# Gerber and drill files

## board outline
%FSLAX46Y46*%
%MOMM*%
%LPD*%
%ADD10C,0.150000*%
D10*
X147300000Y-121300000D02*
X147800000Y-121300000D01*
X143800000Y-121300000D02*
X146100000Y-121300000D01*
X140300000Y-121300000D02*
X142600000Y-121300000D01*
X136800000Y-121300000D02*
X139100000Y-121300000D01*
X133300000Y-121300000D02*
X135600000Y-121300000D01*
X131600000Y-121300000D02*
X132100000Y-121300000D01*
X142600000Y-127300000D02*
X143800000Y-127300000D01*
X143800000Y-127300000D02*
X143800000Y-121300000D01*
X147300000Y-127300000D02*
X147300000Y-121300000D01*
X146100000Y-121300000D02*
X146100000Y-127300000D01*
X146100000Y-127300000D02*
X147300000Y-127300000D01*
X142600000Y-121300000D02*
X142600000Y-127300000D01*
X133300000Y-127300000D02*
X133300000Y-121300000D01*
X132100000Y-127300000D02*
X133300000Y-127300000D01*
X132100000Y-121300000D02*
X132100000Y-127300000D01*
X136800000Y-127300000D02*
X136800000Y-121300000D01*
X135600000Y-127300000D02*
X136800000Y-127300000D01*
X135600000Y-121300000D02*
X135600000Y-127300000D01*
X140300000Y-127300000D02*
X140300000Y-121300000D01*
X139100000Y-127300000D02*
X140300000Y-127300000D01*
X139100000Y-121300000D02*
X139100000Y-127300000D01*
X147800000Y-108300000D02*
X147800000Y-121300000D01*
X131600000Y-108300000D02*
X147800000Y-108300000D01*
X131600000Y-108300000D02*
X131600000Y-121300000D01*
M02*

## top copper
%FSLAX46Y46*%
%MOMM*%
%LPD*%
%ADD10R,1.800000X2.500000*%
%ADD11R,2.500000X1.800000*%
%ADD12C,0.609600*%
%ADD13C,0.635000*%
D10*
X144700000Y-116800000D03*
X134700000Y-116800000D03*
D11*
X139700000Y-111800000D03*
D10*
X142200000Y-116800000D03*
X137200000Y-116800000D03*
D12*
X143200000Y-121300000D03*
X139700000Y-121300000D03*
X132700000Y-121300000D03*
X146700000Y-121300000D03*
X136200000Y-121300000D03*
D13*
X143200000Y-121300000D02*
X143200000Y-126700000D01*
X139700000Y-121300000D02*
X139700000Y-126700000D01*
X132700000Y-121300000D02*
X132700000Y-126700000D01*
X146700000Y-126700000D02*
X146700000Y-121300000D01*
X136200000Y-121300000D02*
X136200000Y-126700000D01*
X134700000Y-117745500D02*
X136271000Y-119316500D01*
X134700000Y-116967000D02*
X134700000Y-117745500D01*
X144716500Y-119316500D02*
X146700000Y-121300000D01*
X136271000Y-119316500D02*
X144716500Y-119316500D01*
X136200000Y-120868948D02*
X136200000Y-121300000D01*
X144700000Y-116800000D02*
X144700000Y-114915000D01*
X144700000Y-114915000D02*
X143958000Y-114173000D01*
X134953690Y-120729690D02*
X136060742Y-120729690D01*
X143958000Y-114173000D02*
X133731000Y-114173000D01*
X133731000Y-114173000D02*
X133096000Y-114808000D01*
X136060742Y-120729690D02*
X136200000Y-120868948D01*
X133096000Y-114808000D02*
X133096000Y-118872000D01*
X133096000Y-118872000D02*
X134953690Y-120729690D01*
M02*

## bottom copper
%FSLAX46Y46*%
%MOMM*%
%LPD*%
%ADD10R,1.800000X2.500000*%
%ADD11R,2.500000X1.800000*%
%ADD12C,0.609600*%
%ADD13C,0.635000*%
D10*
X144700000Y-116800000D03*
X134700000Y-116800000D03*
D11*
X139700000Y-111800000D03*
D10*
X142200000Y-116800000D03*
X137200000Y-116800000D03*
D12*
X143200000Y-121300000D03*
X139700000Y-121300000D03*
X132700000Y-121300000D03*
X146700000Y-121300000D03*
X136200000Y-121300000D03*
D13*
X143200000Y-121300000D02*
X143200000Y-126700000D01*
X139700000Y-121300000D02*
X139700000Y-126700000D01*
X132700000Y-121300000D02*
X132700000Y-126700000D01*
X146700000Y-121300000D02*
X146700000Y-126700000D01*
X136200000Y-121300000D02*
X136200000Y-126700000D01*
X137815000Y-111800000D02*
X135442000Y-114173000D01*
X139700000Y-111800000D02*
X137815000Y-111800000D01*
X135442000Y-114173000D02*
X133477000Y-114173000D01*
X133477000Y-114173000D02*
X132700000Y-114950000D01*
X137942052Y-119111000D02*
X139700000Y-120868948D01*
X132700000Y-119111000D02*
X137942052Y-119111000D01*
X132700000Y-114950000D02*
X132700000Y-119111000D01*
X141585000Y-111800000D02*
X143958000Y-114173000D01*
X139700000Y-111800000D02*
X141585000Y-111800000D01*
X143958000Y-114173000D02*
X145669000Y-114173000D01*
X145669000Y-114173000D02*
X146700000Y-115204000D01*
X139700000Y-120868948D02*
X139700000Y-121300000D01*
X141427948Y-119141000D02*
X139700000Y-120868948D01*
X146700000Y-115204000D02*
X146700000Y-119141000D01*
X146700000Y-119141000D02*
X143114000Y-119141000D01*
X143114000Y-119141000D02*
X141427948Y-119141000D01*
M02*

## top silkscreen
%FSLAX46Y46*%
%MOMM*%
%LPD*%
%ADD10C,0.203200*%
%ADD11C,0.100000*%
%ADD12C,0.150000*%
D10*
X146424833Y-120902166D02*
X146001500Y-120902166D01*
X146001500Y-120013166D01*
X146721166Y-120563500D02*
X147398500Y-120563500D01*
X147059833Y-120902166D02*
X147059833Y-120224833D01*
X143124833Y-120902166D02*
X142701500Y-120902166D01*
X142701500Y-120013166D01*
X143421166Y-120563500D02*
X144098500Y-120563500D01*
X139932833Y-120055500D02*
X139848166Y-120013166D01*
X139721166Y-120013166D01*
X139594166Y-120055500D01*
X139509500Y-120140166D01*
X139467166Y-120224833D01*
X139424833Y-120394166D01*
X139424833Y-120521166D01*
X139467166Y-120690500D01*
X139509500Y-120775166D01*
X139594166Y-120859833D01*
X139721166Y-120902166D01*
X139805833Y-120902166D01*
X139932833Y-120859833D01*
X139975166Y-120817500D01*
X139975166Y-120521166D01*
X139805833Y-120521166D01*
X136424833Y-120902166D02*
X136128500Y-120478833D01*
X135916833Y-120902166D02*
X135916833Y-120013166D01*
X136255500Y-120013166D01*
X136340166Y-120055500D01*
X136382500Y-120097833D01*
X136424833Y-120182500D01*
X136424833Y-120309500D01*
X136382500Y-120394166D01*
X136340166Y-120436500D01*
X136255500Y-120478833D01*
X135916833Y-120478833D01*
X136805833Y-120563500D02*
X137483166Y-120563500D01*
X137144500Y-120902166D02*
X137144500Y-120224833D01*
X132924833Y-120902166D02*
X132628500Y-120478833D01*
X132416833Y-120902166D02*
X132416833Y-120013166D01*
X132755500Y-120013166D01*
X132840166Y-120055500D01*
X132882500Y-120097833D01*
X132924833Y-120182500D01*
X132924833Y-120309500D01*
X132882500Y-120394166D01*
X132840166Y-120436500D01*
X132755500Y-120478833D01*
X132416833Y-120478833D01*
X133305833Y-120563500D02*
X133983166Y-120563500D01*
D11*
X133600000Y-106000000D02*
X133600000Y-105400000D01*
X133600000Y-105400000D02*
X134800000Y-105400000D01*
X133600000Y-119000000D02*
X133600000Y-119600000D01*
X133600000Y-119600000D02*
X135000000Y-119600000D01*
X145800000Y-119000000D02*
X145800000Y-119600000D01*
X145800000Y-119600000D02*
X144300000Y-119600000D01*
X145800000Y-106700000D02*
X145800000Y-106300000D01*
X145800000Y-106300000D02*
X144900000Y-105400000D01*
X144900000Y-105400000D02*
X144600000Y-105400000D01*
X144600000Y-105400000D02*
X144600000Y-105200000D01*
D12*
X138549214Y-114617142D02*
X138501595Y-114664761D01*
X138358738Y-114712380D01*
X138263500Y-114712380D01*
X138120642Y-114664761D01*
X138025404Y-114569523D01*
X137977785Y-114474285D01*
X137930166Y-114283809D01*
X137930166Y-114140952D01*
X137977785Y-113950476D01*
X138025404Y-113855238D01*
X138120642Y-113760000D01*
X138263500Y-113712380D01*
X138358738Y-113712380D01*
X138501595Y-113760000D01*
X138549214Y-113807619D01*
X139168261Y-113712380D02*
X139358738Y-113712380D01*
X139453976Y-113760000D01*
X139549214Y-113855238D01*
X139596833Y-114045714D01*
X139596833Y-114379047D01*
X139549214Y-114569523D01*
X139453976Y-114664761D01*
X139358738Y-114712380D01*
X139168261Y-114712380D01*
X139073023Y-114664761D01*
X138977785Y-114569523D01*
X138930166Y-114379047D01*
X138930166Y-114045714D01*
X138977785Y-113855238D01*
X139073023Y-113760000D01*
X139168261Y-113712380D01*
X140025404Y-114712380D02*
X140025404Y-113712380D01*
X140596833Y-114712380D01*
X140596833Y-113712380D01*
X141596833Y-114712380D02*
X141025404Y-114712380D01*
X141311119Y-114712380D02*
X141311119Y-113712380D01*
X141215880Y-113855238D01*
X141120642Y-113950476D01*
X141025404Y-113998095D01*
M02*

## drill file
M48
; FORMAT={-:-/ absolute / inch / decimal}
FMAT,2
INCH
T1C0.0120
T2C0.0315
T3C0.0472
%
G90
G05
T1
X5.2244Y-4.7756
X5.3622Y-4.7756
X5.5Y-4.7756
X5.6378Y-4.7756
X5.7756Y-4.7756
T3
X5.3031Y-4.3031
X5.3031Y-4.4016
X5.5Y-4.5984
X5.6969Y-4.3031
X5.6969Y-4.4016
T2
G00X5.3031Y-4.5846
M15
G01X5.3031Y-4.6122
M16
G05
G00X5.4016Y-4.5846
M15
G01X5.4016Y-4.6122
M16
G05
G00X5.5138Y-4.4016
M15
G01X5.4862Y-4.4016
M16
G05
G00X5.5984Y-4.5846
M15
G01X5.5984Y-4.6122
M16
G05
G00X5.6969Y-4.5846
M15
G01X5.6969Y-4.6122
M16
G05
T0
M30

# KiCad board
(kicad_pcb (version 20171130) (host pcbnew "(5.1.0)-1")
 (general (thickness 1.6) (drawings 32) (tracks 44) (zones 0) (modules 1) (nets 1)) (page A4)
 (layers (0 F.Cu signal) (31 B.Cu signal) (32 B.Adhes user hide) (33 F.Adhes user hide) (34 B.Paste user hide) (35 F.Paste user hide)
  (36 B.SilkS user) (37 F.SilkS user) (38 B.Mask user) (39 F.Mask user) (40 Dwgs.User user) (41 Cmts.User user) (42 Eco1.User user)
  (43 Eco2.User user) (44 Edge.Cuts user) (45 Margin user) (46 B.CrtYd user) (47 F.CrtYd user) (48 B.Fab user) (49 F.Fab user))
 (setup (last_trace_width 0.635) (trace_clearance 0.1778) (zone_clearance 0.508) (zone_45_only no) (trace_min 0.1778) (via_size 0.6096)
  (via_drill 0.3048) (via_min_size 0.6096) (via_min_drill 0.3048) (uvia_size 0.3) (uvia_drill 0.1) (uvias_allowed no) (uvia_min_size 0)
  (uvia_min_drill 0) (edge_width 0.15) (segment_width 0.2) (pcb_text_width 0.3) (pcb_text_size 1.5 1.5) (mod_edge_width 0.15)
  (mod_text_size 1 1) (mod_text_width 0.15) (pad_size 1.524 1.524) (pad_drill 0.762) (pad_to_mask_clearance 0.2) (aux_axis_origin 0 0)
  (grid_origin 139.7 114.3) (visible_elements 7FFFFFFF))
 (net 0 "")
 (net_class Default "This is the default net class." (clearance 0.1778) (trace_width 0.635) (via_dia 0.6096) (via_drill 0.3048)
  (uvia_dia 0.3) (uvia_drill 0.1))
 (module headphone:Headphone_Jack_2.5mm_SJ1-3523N (layer F.Cu) (at 139.7 116.8 270)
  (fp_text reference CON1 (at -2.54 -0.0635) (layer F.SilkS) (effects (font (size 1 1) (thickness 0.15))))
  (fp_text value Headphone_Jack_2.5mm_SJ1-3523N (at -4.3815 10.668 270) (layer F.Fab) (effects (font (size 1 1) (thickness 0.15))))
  (fp_line (start -10.8 6.1) (end -11.4 6.1) (layer F.SilkS) (width 0.1))
  (fp_line (start -11.4 6.1) (end -11.4 4.9) (layer F.SilkS) (width 0.1))
  (fp_line (start 2.2 6.1) (end 2.8 6.1) (layer F.SilkS) (width 0.1))
  (fp_line (start 2.8 6.1) (end 2.8 4.7) (layer F.SilkS) (width 0.1))
  (fp_line (start 2.2 -6.1) (end 2.8 -6.1) (layer F.SilkS) (width 0.1))
  (fp_line (start 2.8 -6.1) (end 2.8 -4.6) (layer F.SilkS) (width 0.1))
  (fp_line (start -10.1 -6.1) (end -10.5 -6.1) (layer F.SilkS) (width 0.1))
  (fp_line (start -10.5 -6.1) (end -11.4 -5.2) (layer F.SilkS) (width 0.1))
  (fp_line (start -11.4 -5.2) (end -11.4 -4.9) (layer F.SilkS) (width 0.1))
  (fp_line (start -11.4 -4.9) (end -11.6 -4.9) (layer F.SilkS) (width 0.1))
  (pad 3 thru_hole rect (at 0 -5 270) (size 2.5 1.8) (drill oval 1.5 0.8) (layers *.Cu *.Mask))
  (pad 2 thru_hole rect (at 0 5 270) (size 2.5 1.8) (drill oval 1.5 0.8) (layers *.Cu *.Mask))
  (pad 1 thru_hole rect (at -5 0 270) (size 1.8 2.5) (drill oval 0.8 1.5) (layers *.Cu *.Mask))
  (pad "" np_thru_hole circle (at 0 0 270) (size 1.2 1.2) (drill 1.2) (layers *.Cu *.Mask))
  (pad "" np_thru_hole circle (at -5 -5 270) (size 1.2 1.2) (drill 1.2) (layers *.Cu *.Mask))
  (pad "" np_thru_hole circle (at -7.5 -5 270) (size 1.2 1.2) (drill 1.2) (layers *.Cu *.Mask))
  (pad "" np_thru_hole circle (at -5 5 270) (size 1.2 1.2) (drill 1.2) (layers *.Cu *.Mask))
  (pad "" np_thru_hole circle (at -7.5 5 270) (size 1.2 1.2) (drill 1.2) (layers *.Cu *.Mask))
  (pad 11 thru_hole rect (at 0 -2.5 270) (size 2.5 1.8) (drill oval 1.5 0.8) (layers *.Cu *.Mask))
  (pad 10 thru_hole rect (at 0 2.5 270) (size 2.5 1.8) (drill oval 1.5 0.8) (layers *.Cu *.Mask)))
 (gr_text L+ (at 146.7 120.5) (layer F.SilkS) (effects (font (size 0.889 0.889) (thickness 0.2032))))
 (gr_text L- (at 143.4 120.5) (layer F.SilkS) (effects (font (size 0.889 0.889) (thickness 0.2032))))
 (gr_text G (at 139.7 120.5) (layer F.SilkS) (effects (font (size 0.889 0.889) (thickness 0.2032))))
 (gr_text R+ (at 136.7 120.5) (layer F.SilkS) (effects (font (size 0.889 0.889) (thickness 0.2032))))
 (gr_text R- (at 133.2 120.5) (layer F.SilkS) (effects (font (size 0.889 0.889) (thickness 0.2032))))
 (gr_line (start 147.3 121.3) (end 147.8 121.3) (layer Edge.Cuts) (width 0.15))
 (gr_line (start 143.8 121.3) (end 146.1 121.3) (layer Edge.Cuts) (width 0.15))
 (gr_line (start 140.3 121.3) (end 142.6 121.3) (layer Edge.Cuts) (width 0.15))
 (gr_line (start 136.8 121.3) (end 139.1 121.3) (layer Edge.Cuts) (width 0.15))
 (gr_line (start 133.3 121.3) (end 135.6 121.3) (layer Edge.Cuts) (width 0.15))
 (gr_line (start 131.6 121.3) (end 132.1 121.3) (layer Edge.Cuts) (width 0.15))
 (gr_line (start 142.6 127.3) (end 143.8 127.3) (layer Edge.Cuts) (width 0.15))
 (gr_line (start 143.8 127.3) (end 143.8 121.3) (layer Edge.Cuts) (width 0.15))
 (gr_line (start 147.3 127.3) (end 147.3 121.3) (layer Edge.Cuts) (width 0.15))
 (gr_line (start 146.1 121.3) (end 146.1 127.3) (layer Edge.Cuts) (width 0.15))
 (gr_line (start 146.1 127.3) (end 147.3 127.3) (layer Edge.Cuts) (width 0.15))
 (gr_line (start 142.6 121.3) (end 142.6 127.3) (layer Edge.Cuts) (width 0.15))
 (gr_line (start 133.3 127.3) (end 133.3 121.3) (layer Edge.Cuts) (width 0.15))
 (gr_line (start 132.1 127.3) (end 133.3 127.3) (layer Edge.Cuts) (width 0.15))
 (gr_line (start 132.1 121.3) (end 132.1 127.3) (layer Edge.Cuts) (width 0.15))
 (gr_line (start 136.8 127.3) (end 136.8 121.3) (layer Edge.Cuts) (width 0.15))
 (gr_line (start 135.6 127.3) (end 136.8 127.3) (layer Edge.Cuts) (width 0.15))
 (gr_line (start 135.6 121.3) (end 135.6 127.3) (layer Edge.Cuts) (width 0.15))
 (gr_line (start 140.3 127.3) (end 140.3 121.3) (layer Edge.Cuts) (width 0.15))
 (gr_line (start 139.1 127.3) (end 140.3 127.3) (layer Edge.Cuts) (width 0.15))
 (gr_line (start 139.1 121.3) (end 139.1 127.3) (layer Edge.Cuts) (width 0.15))
 (gr_line (start 147.8 108.3) (end 147.8 121.3) (layer Edge.Cuts) (width 0.15))
 (gr_line (start 131.6 108.3) (end 147.8 108.3) (layer Edge.Cuts) (width 0.15))
 (gr_line (start 131.6 108.3) (end 131.6 121.3) (layer Edge.Cuts) (width 0.15))
 (segment (start 143.2 121.3) (end 143.2 126.7) (width 0.635) (layer F.Cu) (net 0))
 (via (at 143.2 121.3) (size 0.6096) (drill 0.3048) (layers F.Cu B.Cu) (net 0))
 (segment (start 143.2 121.3) (end 143.2 126.7) (width 0.635) (layer B.Cu) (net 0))
 (segment (start 139.7 121.3) (end 139.7 126.7) (width 0.635) (layer F.Cu) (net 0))
 (segment (start 139.7 121.3) (end 139.7 126.7) (width 0.635) (layer B.Cu) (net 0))
 (via (at 139.7 121.3) (size 0.6096) (drill 0.3048) (layers F.Cu B.Cu) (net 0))
 (segment (start 132.7 121.3) (end 132.7 126.7) (width 0.635) (layer F.Cu) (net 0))
 (segment (start 132.7 121.3) (end 132.7 126.7) (width 0.635) (layer B.Cu) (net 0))
 (via (at 132.7 121.3) (size 0.6096) (drill 0.3048) (layers F.Cu B.Cu) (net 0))
 (segment (start 146.7 121.3) (end 146.7 126.7) (width 0.635) (layer B.Cu) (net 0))
 (segment (start 146.7 126.7) (end 146.7 121.3) (width 0.635) (layer F.Cu) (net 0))
 (via (at 146.7 121.3) (size 0.6096) (drill 0.3048) (layers F.Cu B.Cu) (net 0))
 (segment (start 136.2 121.3) (end 136.2 126.7) (width 0.635) (layer B.Cu) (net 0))
 (segment (start 136.2 121.3) (end 136.2 126.7) (width 0.635) (layer F.Cu) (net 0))
 (via (at 136.2 121.3) (size 0.6096) (drill 0.3048) (layers F.Cu B.Cu) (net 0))
 (segment (start 134.7 117.7455) (end 136.271 119.3165) (width 0.635) (layer F.Cu) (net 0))
 (segment (start 134.7 116.967) (end 134.7 117.7455) (width 0.635) (layer F.Cu) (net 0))
 (segment (start 144.7165 119.3165) (end 146.7 121.3) (width 0.635) (layer F.Cu) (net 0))
 (segment (start 136.271 119.3165) (end 144.7165 119.3165) (width 0.635) (layer F.Cu) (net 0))
 (segment (start 136.2 120.868948) (end 136.2 121.3) (width 0.635) (layer F.Cu) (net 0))
 (segment (start 144.7 116.8) (end 144.7 114.915) (width 0.635) (layer F.Cu) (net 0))
 (segment (start 144.7 114.915) (end 143.958 114.173) (width 0.635) (layer F.Cu) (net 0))
 (segment (start 134.95369 120.72969) (end 136.060742 120.72969) (width 0.635) (layer F.Cu) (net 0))
 (segment (start 143.958 114.173) (end 133.731 114.173) (width 0.635) (layer F.Cu) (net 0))
 (segment (start 133.731 114.173) (end 133.096 114.808) (width 0.635) (layer F.Cu) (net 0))
 (segment (start 136.060742 120.72969) (end 136.2 120.868948) (width 0.635) (layer F.Cu) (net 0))
 (segment (start 133.096 114.808) (end 133.096 118.872) (width 0.635) (layer F.Cu) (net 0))
 (segment (start 133.096 118.872) (end 134.95369 120.72969) (width 0.635) (layer F.Cu) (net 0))
 (segment (start 137.815 111.8) (end 135.442 114.173) (width 0.635) (layer B.Cu) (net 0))
 (segment (start 139.7 111.8) (end 137.815 111.8) (width 0.635) (layer B.Cu) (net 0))
 (segment (start 135.442 114.173) (end 133.477 114.173) (width 0.635) (layer B.Cu) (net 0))
 (segment (start 133.477 114.173) (end 132.7 114.95) (width 0.635) (layer B.Cu) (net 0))
 (segment (start 137.942052 119.111) (end 139.7 120.868948) (width 0.635) (layer B.Cu) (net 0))
 (segment (start 132.7 119.111) (end 137.942052 119.111) (width 0.635) (layer B.Cu) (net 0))
 (segment (start 132.7 114.95) (end 132.7 119.111) (width 0.635) (layer B.Cu) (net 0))
 (segment (start 141.585 111.8) (end 143.958 114.173) (width 0.635) (layer B.Cu) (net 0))
 (segment (start 139.7 111.8) (end 141.585 111.8) (width 0.635) (layer B.Cu) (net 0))
 (segment (start 143.958 114.173) (end 145.669 114.173) (width 0.635) (layer B.Cu) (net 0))
 (segment (start 145.669 114.173) (end 146.7 115.204) (width 0.635) (layer B.Cu) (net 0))
 (segment (start 139.7 120.868948) (end 139.7 121.3) (width 0.635) (layer B.Cu) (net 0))
 (segment (start 141.427948 119.141) (end 139.7 120.868948) (width 0.635) (layer B.Cu) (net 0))
 (segment (start 146.7 115.204) (end 146.7 119.141) (width 0.635) (layer B.Cu) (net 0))
 (segment (start 146.7 119.141) (end 143.114 119.141) (width 0.635) (layer B.Cu) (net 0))
 (segment (start 143.114 119.141) (end 141.427948 119.141) (width 0.635) (layer B.Cu) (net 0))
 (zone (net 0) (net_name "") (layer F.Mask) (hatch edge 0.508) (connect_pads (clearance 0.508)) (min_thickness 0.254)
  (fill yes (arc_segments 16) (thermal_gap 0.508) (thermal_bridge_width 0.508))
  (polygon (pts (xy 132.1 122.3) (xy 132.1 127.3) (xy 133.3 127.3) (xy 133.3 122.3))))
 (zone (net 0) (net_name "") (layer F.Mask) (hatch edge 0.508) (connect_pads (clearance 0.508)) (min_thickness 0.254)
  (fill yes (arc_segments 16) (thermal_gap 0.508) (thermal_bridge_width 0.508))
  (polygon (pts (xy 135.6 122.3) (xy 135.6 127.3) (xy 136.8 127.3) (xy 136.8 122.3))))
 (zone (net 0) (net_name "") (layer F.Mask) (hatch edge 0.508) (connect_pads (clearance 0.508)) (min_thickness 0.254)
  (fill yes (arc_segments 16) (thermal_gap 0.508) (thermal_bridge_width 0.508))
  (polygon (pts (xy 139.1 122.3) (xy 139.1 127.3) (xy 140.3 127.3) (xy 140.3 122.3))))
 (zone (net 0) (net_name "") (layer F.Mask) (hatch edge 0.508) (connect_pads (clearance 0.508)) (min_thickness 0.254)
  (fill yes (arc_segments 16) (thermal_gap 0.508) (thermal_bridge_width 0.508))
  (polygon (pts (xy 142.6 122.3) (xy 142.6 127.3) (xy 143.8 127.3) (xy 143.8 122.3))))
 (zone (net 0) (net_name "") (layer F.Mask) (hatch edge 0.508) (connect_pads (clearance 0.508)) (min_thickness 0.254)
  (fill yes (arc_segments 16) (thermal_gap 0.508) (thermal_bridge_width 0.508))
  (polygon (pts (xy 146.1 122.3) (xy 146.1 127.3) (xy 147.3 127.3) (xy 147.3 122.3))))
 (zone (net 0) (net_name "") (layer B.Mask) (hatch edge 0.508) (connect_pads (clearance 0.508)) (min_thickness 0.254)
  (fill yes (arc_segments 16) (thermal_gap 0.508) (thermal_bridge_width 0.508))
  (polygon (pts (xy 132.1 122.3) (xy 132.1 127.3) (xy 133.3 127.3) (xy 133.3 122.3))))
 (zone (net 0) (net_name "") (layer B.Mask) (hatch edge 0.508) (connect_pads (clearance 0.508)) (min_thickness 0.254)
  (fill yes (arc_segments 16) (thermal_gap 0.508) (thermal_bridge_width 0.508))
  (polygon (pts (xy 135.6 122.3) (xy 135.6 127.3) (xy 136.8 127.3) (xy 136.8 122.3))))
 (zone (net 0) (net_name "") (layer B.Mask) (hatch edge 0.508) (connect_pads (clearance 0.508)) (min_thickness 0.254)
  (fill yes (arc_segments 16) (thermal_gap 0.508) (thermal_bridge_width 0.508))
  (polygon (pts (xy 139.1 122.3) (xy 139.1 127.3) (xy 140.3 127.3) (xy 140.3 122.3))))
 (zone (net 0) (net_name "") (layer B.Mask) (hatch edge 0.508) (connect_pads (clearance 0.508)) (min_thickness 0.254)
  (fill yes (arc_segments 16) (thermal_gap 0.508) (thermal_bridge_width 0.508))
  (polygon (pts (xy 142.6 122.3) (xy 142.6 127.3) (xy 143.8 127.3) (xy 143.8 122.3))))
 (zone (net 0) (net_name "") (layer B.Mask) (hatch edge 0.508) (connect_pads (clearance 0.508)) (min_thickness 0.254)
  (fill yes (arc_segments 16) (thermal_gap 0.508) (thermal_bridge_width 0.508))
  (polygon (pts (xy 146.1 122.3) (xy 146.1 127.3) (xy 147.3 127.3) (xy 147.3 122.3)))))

